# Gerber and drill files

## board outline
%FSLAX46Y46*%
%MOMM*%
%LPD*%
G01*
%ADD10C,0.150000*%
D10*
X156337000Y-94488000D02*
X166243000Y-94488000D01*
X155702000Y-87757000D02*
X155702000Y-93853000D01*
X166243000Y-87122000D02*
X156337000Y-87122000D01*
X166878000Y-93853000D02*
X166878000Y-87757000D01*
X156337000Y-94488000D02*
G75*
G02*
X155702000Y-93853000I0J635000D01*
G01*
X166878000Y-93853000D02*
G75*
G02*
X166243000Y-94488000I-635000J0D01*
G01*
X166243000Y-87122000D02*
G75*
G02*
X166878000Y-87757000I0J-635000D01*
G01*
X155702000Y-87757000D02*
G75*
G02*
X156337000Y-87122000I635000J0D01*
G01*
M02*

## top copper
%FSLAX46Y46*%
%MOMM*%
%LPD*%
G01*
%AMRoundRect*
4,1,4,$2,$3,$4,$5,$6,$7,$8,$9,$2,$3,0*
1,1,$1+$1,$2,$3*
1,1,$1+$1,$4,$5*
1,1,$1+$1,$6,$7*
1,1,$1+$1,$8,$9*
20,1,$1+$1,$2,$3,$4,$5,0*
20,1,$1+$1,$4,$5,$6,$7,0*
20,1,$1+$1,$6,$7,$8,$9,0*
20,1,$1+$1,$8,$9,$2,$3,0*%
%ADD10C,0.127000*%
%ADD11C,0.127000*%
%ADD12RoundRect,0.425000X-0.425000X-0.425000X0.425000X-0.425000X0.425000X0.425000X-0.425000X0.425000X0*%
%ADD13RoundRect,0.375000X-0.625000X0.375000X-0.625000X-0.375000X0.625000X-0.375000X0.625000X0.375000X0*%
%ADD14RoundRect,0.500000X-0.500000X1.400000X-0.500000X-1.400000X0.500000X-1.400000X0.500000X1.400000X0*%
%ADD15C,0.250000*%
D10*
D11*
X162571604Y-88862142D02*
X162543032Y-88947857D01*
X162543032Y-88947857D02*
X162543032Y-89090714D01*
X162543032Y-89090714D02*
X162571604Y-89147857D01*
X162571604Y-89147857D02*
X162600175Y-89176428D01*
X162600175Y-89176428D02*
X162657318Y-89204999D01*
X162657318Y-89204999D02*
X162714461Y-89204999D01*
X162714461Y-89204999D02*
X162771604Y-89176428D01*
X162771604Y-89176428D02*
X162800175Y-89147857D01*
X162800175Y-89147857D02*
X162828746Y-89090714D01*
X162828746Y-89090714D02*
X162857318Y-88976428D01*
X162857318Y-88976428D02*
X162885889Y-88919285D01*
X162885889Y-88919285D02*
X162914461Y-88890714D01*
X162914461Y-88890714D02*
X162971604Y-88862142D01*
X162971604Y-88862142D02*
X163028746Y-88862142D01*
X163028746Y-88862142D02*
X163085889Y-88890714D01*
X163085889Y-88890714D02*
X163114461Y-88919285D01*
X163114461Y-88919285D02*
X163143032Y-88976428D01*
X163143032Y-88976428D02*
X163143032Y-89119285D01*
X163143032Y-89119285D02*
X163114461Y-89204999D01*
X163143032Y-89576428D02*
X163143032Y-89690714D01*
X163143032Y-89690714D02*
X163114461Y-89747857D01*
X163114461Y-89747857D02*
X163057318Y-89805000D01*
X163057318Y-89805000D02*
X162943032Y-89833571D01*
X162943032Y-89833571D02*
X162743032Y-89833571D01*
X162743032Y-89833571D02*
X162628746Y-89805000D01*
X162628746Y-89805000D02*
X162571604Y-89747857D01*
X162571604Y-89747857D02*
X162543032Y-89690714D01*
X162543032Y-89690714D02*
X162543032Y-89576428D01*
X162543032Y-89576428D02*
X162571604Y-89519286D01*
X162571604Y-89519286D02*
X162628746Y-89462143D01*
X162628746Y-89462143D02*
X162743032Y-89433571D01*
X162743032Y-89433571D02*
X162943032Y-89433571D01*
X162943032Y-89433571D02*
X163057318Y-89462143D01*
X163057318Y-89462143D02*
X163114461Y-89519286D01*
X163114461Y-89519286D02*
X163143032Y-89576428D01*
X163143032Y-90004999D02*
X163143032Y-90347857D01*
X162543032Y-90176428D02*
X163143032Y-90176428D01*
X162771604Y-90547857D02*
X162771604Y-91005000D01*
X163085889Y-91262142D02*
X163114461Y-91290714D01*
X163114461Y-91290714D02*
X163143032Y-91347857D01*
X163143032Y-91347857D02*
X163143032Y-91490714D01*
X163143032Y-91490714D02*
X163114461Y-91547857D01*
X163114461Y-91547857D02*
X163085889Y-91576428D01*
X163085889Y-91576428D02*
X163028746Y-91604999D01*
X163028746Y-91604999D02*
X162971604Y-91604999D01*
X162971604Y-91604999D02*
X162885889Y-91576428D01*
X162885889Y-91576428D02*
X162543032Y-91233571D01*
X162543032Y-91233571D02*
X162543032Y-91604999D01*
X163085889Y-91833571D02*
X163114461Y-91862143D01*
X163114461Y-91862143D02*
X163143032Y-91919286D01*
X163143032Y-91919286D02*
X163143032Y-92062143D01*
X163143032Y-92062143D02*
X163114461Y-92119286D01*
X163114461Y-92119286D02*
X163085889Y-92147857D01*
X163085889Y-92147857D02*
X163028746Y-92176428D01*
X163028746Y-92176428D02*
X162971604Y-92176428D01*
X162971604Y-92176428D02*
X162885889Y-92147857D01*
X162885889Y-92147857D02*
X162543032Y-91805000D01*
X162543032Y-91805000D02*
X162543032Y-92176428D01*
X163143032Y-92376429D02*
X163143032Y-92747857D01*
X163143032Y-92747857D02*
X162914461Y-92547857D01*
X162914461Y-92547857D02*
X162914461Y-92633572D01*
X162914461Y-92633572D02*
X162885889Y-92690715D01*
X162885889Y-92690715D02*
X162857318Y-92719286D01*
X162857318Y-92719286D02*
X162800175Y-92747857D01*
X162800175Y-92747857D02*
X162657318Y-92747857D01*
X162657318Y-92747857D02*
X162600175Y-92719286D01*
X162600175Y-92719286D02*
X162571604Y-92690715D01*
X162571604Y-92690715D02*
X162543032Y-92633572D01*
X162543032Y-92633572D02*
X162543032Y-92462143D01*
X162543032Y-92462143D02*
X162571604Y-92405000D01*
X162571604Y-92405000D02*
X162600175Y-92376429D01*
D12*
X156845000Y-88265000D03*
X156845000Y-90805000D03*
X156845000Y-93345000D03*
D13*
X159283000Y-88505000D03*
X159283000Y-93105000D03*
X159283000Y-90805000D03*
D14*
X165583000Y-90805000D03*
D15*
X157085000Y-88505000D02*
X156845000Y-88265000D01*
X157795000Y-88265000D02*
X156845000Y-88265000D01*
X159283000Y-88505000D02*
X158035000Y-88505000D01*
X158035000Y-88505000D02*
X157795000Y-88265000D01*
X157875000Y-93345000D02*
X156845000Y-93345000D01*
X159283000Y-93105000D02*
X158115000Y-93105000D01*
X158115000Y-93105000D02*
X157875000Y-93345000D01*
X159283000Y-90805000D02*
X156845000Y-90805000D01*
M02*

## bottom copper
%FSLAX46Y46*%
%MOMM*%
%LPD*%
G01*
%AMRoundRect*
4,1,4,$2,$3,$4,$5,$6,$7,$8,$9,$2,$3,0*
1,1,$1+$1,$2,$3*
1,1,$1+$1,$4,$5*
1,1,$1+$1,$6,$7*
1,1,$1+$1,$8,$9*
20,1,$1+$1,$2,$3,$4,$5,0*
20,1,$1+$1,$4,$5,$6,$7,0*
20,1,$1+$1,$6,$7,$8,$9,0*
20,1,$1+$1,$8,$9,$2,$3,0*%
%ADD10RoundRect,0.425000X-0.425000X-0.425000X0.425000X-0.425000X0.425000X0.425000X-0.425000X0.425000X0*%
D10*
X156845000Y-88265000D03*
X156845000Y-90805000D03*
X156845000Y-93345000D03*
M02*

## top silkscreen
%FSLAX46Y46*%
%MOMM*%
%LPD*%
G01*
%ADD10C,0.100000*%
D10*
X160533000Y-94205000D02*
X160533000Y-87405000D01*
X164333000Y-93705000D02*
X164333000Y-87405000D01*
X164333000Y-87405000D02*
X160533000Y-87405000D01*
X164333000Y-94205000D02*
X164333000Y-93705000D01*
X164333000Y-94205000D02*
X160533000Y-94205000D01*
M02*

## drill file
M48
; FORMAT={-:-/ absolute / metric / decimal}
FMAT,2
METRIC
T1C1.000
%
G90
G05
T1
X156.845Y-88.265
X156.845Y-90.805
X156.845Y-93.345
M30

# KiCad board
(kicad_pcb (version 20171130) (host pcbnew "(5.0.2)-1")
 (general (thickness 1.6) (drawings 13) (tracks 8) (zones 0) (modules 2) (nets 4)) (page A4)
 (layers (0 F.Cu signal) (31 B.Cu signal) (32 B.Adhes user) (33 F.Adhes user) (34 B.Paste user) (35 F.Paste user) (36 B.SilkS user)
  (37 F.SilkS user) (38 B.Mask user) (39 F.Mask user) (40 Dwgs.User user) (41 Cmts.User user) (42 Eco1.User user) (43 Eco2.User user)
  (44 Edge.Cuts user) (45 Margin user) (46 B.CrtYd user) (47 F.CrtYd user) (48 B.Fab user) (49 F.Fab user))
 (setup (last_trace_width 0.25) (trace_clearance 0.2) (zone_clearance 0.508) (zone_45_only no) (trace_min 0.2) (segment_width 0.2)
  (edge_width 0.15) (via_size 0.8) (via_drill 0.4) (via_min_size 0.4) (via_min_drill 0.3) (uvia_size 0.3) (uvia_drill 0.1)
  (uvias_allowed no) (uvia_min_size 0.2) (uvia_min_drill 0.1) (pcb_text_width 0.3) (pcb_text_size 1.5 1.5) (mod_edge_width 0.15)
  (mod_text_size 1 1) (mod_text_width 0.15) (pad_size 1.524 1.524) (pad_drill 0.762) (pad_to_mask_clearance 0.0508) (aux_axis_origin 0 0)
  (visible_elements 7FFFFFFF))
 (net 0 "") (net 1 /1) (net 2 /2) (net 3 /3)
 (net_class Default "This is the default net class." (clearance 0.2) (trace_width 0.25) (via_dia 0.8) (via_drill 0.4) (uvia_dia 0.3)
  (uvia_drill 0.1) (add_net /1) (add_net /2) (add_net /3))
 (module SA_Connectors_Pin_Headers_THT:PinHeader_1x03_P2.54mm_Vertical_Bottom (layer F.Cu) (at 156.845 88.265)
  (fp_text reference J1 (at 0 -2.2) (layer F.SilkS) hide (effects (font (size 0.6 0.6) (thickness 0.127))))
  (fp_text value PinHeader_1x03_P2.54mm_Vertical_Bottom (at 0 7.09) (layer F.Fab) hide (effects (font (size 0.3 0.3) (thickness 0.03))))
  (pad 1 thru_hole roundrect (at 0 0) (size 1.7 1.7) (drill 1) (layers *.Cu *.Mask) (roundrect_rratio 0.25) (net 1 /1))
  (pad 2 thru_hole roundrect (at 0 2.54) (size 1.7 1.7) (drill 1) (layers *.Cu *.Mask) (roundrect_rratio 0.25) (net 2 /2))
  (pad 3 thru_hole roundrect (at 0 5.08) (size 1.7 1.7) (drill 1) (layers *.Cu *.Mask) (roundrect_rratio 0.25) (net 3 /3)))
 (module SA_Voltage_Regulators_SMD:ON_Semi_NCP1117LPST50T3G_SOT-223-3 (layer F.Cu) (at 162.433 90.805 270)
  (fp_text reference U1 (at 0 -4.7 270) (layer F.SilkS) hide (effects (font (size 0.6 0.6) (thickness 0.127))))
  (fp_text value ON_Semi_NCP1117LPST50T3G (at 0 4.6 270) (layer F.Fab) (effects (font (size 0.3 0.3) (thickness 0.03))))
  (fp_line (start 3.4 1.9) (end -3.4 1.9) (layer F.SilkS) (width 0.1))
  (fp_line (start 2.9 -1.9) (end -3.4 -1.9) (layer F.SilkS) (width 0.1))
  (fp_line (start -3.4 -1.9) (end -3.4 1.9) (layer F.SilkS) (width 0.1))
  (fp_line (start 3.4 -1.9) (end 2.9 -1.9) (layer F.SilkS) (width 0.1))
  (fp_line (start 3.4 -1.9) (end 3.4 1.9) (layer F.SilkS) (width 0.1))
  (pad 1 smd roundrect (at -2.3 3.15 270) (size 1.5 2) (layers F.Cu F.Paste F.Mask) (roundrect_rratio 0.25) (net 1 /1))
  (pad 3 smd roundrect (at 2.3 3.15 270) (size 1.5 2) (layers F.Cu F.Paste F.Mask) (roundrect_rratio 0.25) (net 3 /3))
  (pad 2 smd roundrect (at 0 3.15 270) (size 1.5 2) (layers F.Cu F.Paste F.Mask) (roundrect_rratio 0.25) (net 2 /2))
  (pad 2 smd roundrect (at 0 -3.15 270) (size 3.8 2) (layers F.Cu F.Paste F.Mask) (roundrect_rratio 0.25) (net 2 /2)))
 (gr_line (start 156.337 94.488) (end 166.243 94.488) (layer Edge.Cuts) (width 0.15))
 (gr_line (start 155.702 87.757) (end 155.702 93.853) (layer Edge.Cuts) (width 0.15))
 (gr_line (start 166.243 87.122) (end 156.337 87.122) (layer Edge.Cuts) (width 0.15))
 (gr_line (start 166.878 93.853) (end 166.878 87.757) (layer Edge.Cuts) (width 0.15))
 (gr_arc (start 156.337 93.853) (end 155.702 93.853) (angle -90) (layer Edge.Cuts) (width 0.15))
 (gr_arc (start 166.243 93.853) (end 166.243 94.488) (angle -90) (layer Edge.Cuts) (width 0.15))
 (gr_arc (start 166.243 87.757) (end 166.878 87.757) (angle -90) (layer Edge.Cuts) (width 0.15))
 (gr_arc (start 156.337 87.757) (end 156.337 87.122) (angle -90) (layer Edge.Cuts) (width 0.15))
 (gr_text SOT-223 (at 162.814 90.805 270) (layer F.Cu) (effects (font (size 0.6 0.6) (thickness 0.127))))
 (segment (start 157.085 88.505) (end 156.845 88.265) (width 0.25) (layer F.Cu) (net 1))
 (segment (start 157.795 88.265) (end 156.845 88.265) (width 0.25) (layer F.Cu) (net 1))
 (segment (start 159.283 88.505) (end 158.035 88.505) (width 0.25) (layer F.Cu) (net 1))
 (segment (start 158.035 88.505) (end 157.795 88.265) (width 0.25) (layer F.Cu) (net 1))
 (segment (start 157.875 93.345) (end 156.845 93.345) (width 0.25) (layer F.Cu) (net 3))
 (segment (start 159.283 93.105) (end 158.115 93.105) (width 0.25) (layer F.Cu) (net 3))
 (segment (start 158.115 93.105) (end 157.875 93.345) (width 0.25) (layer F.Cu) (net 3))
 (segment (start 159.283 90.805) (end 156.845 90.805) (width 0.25) (layer F.Cu) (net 2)))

